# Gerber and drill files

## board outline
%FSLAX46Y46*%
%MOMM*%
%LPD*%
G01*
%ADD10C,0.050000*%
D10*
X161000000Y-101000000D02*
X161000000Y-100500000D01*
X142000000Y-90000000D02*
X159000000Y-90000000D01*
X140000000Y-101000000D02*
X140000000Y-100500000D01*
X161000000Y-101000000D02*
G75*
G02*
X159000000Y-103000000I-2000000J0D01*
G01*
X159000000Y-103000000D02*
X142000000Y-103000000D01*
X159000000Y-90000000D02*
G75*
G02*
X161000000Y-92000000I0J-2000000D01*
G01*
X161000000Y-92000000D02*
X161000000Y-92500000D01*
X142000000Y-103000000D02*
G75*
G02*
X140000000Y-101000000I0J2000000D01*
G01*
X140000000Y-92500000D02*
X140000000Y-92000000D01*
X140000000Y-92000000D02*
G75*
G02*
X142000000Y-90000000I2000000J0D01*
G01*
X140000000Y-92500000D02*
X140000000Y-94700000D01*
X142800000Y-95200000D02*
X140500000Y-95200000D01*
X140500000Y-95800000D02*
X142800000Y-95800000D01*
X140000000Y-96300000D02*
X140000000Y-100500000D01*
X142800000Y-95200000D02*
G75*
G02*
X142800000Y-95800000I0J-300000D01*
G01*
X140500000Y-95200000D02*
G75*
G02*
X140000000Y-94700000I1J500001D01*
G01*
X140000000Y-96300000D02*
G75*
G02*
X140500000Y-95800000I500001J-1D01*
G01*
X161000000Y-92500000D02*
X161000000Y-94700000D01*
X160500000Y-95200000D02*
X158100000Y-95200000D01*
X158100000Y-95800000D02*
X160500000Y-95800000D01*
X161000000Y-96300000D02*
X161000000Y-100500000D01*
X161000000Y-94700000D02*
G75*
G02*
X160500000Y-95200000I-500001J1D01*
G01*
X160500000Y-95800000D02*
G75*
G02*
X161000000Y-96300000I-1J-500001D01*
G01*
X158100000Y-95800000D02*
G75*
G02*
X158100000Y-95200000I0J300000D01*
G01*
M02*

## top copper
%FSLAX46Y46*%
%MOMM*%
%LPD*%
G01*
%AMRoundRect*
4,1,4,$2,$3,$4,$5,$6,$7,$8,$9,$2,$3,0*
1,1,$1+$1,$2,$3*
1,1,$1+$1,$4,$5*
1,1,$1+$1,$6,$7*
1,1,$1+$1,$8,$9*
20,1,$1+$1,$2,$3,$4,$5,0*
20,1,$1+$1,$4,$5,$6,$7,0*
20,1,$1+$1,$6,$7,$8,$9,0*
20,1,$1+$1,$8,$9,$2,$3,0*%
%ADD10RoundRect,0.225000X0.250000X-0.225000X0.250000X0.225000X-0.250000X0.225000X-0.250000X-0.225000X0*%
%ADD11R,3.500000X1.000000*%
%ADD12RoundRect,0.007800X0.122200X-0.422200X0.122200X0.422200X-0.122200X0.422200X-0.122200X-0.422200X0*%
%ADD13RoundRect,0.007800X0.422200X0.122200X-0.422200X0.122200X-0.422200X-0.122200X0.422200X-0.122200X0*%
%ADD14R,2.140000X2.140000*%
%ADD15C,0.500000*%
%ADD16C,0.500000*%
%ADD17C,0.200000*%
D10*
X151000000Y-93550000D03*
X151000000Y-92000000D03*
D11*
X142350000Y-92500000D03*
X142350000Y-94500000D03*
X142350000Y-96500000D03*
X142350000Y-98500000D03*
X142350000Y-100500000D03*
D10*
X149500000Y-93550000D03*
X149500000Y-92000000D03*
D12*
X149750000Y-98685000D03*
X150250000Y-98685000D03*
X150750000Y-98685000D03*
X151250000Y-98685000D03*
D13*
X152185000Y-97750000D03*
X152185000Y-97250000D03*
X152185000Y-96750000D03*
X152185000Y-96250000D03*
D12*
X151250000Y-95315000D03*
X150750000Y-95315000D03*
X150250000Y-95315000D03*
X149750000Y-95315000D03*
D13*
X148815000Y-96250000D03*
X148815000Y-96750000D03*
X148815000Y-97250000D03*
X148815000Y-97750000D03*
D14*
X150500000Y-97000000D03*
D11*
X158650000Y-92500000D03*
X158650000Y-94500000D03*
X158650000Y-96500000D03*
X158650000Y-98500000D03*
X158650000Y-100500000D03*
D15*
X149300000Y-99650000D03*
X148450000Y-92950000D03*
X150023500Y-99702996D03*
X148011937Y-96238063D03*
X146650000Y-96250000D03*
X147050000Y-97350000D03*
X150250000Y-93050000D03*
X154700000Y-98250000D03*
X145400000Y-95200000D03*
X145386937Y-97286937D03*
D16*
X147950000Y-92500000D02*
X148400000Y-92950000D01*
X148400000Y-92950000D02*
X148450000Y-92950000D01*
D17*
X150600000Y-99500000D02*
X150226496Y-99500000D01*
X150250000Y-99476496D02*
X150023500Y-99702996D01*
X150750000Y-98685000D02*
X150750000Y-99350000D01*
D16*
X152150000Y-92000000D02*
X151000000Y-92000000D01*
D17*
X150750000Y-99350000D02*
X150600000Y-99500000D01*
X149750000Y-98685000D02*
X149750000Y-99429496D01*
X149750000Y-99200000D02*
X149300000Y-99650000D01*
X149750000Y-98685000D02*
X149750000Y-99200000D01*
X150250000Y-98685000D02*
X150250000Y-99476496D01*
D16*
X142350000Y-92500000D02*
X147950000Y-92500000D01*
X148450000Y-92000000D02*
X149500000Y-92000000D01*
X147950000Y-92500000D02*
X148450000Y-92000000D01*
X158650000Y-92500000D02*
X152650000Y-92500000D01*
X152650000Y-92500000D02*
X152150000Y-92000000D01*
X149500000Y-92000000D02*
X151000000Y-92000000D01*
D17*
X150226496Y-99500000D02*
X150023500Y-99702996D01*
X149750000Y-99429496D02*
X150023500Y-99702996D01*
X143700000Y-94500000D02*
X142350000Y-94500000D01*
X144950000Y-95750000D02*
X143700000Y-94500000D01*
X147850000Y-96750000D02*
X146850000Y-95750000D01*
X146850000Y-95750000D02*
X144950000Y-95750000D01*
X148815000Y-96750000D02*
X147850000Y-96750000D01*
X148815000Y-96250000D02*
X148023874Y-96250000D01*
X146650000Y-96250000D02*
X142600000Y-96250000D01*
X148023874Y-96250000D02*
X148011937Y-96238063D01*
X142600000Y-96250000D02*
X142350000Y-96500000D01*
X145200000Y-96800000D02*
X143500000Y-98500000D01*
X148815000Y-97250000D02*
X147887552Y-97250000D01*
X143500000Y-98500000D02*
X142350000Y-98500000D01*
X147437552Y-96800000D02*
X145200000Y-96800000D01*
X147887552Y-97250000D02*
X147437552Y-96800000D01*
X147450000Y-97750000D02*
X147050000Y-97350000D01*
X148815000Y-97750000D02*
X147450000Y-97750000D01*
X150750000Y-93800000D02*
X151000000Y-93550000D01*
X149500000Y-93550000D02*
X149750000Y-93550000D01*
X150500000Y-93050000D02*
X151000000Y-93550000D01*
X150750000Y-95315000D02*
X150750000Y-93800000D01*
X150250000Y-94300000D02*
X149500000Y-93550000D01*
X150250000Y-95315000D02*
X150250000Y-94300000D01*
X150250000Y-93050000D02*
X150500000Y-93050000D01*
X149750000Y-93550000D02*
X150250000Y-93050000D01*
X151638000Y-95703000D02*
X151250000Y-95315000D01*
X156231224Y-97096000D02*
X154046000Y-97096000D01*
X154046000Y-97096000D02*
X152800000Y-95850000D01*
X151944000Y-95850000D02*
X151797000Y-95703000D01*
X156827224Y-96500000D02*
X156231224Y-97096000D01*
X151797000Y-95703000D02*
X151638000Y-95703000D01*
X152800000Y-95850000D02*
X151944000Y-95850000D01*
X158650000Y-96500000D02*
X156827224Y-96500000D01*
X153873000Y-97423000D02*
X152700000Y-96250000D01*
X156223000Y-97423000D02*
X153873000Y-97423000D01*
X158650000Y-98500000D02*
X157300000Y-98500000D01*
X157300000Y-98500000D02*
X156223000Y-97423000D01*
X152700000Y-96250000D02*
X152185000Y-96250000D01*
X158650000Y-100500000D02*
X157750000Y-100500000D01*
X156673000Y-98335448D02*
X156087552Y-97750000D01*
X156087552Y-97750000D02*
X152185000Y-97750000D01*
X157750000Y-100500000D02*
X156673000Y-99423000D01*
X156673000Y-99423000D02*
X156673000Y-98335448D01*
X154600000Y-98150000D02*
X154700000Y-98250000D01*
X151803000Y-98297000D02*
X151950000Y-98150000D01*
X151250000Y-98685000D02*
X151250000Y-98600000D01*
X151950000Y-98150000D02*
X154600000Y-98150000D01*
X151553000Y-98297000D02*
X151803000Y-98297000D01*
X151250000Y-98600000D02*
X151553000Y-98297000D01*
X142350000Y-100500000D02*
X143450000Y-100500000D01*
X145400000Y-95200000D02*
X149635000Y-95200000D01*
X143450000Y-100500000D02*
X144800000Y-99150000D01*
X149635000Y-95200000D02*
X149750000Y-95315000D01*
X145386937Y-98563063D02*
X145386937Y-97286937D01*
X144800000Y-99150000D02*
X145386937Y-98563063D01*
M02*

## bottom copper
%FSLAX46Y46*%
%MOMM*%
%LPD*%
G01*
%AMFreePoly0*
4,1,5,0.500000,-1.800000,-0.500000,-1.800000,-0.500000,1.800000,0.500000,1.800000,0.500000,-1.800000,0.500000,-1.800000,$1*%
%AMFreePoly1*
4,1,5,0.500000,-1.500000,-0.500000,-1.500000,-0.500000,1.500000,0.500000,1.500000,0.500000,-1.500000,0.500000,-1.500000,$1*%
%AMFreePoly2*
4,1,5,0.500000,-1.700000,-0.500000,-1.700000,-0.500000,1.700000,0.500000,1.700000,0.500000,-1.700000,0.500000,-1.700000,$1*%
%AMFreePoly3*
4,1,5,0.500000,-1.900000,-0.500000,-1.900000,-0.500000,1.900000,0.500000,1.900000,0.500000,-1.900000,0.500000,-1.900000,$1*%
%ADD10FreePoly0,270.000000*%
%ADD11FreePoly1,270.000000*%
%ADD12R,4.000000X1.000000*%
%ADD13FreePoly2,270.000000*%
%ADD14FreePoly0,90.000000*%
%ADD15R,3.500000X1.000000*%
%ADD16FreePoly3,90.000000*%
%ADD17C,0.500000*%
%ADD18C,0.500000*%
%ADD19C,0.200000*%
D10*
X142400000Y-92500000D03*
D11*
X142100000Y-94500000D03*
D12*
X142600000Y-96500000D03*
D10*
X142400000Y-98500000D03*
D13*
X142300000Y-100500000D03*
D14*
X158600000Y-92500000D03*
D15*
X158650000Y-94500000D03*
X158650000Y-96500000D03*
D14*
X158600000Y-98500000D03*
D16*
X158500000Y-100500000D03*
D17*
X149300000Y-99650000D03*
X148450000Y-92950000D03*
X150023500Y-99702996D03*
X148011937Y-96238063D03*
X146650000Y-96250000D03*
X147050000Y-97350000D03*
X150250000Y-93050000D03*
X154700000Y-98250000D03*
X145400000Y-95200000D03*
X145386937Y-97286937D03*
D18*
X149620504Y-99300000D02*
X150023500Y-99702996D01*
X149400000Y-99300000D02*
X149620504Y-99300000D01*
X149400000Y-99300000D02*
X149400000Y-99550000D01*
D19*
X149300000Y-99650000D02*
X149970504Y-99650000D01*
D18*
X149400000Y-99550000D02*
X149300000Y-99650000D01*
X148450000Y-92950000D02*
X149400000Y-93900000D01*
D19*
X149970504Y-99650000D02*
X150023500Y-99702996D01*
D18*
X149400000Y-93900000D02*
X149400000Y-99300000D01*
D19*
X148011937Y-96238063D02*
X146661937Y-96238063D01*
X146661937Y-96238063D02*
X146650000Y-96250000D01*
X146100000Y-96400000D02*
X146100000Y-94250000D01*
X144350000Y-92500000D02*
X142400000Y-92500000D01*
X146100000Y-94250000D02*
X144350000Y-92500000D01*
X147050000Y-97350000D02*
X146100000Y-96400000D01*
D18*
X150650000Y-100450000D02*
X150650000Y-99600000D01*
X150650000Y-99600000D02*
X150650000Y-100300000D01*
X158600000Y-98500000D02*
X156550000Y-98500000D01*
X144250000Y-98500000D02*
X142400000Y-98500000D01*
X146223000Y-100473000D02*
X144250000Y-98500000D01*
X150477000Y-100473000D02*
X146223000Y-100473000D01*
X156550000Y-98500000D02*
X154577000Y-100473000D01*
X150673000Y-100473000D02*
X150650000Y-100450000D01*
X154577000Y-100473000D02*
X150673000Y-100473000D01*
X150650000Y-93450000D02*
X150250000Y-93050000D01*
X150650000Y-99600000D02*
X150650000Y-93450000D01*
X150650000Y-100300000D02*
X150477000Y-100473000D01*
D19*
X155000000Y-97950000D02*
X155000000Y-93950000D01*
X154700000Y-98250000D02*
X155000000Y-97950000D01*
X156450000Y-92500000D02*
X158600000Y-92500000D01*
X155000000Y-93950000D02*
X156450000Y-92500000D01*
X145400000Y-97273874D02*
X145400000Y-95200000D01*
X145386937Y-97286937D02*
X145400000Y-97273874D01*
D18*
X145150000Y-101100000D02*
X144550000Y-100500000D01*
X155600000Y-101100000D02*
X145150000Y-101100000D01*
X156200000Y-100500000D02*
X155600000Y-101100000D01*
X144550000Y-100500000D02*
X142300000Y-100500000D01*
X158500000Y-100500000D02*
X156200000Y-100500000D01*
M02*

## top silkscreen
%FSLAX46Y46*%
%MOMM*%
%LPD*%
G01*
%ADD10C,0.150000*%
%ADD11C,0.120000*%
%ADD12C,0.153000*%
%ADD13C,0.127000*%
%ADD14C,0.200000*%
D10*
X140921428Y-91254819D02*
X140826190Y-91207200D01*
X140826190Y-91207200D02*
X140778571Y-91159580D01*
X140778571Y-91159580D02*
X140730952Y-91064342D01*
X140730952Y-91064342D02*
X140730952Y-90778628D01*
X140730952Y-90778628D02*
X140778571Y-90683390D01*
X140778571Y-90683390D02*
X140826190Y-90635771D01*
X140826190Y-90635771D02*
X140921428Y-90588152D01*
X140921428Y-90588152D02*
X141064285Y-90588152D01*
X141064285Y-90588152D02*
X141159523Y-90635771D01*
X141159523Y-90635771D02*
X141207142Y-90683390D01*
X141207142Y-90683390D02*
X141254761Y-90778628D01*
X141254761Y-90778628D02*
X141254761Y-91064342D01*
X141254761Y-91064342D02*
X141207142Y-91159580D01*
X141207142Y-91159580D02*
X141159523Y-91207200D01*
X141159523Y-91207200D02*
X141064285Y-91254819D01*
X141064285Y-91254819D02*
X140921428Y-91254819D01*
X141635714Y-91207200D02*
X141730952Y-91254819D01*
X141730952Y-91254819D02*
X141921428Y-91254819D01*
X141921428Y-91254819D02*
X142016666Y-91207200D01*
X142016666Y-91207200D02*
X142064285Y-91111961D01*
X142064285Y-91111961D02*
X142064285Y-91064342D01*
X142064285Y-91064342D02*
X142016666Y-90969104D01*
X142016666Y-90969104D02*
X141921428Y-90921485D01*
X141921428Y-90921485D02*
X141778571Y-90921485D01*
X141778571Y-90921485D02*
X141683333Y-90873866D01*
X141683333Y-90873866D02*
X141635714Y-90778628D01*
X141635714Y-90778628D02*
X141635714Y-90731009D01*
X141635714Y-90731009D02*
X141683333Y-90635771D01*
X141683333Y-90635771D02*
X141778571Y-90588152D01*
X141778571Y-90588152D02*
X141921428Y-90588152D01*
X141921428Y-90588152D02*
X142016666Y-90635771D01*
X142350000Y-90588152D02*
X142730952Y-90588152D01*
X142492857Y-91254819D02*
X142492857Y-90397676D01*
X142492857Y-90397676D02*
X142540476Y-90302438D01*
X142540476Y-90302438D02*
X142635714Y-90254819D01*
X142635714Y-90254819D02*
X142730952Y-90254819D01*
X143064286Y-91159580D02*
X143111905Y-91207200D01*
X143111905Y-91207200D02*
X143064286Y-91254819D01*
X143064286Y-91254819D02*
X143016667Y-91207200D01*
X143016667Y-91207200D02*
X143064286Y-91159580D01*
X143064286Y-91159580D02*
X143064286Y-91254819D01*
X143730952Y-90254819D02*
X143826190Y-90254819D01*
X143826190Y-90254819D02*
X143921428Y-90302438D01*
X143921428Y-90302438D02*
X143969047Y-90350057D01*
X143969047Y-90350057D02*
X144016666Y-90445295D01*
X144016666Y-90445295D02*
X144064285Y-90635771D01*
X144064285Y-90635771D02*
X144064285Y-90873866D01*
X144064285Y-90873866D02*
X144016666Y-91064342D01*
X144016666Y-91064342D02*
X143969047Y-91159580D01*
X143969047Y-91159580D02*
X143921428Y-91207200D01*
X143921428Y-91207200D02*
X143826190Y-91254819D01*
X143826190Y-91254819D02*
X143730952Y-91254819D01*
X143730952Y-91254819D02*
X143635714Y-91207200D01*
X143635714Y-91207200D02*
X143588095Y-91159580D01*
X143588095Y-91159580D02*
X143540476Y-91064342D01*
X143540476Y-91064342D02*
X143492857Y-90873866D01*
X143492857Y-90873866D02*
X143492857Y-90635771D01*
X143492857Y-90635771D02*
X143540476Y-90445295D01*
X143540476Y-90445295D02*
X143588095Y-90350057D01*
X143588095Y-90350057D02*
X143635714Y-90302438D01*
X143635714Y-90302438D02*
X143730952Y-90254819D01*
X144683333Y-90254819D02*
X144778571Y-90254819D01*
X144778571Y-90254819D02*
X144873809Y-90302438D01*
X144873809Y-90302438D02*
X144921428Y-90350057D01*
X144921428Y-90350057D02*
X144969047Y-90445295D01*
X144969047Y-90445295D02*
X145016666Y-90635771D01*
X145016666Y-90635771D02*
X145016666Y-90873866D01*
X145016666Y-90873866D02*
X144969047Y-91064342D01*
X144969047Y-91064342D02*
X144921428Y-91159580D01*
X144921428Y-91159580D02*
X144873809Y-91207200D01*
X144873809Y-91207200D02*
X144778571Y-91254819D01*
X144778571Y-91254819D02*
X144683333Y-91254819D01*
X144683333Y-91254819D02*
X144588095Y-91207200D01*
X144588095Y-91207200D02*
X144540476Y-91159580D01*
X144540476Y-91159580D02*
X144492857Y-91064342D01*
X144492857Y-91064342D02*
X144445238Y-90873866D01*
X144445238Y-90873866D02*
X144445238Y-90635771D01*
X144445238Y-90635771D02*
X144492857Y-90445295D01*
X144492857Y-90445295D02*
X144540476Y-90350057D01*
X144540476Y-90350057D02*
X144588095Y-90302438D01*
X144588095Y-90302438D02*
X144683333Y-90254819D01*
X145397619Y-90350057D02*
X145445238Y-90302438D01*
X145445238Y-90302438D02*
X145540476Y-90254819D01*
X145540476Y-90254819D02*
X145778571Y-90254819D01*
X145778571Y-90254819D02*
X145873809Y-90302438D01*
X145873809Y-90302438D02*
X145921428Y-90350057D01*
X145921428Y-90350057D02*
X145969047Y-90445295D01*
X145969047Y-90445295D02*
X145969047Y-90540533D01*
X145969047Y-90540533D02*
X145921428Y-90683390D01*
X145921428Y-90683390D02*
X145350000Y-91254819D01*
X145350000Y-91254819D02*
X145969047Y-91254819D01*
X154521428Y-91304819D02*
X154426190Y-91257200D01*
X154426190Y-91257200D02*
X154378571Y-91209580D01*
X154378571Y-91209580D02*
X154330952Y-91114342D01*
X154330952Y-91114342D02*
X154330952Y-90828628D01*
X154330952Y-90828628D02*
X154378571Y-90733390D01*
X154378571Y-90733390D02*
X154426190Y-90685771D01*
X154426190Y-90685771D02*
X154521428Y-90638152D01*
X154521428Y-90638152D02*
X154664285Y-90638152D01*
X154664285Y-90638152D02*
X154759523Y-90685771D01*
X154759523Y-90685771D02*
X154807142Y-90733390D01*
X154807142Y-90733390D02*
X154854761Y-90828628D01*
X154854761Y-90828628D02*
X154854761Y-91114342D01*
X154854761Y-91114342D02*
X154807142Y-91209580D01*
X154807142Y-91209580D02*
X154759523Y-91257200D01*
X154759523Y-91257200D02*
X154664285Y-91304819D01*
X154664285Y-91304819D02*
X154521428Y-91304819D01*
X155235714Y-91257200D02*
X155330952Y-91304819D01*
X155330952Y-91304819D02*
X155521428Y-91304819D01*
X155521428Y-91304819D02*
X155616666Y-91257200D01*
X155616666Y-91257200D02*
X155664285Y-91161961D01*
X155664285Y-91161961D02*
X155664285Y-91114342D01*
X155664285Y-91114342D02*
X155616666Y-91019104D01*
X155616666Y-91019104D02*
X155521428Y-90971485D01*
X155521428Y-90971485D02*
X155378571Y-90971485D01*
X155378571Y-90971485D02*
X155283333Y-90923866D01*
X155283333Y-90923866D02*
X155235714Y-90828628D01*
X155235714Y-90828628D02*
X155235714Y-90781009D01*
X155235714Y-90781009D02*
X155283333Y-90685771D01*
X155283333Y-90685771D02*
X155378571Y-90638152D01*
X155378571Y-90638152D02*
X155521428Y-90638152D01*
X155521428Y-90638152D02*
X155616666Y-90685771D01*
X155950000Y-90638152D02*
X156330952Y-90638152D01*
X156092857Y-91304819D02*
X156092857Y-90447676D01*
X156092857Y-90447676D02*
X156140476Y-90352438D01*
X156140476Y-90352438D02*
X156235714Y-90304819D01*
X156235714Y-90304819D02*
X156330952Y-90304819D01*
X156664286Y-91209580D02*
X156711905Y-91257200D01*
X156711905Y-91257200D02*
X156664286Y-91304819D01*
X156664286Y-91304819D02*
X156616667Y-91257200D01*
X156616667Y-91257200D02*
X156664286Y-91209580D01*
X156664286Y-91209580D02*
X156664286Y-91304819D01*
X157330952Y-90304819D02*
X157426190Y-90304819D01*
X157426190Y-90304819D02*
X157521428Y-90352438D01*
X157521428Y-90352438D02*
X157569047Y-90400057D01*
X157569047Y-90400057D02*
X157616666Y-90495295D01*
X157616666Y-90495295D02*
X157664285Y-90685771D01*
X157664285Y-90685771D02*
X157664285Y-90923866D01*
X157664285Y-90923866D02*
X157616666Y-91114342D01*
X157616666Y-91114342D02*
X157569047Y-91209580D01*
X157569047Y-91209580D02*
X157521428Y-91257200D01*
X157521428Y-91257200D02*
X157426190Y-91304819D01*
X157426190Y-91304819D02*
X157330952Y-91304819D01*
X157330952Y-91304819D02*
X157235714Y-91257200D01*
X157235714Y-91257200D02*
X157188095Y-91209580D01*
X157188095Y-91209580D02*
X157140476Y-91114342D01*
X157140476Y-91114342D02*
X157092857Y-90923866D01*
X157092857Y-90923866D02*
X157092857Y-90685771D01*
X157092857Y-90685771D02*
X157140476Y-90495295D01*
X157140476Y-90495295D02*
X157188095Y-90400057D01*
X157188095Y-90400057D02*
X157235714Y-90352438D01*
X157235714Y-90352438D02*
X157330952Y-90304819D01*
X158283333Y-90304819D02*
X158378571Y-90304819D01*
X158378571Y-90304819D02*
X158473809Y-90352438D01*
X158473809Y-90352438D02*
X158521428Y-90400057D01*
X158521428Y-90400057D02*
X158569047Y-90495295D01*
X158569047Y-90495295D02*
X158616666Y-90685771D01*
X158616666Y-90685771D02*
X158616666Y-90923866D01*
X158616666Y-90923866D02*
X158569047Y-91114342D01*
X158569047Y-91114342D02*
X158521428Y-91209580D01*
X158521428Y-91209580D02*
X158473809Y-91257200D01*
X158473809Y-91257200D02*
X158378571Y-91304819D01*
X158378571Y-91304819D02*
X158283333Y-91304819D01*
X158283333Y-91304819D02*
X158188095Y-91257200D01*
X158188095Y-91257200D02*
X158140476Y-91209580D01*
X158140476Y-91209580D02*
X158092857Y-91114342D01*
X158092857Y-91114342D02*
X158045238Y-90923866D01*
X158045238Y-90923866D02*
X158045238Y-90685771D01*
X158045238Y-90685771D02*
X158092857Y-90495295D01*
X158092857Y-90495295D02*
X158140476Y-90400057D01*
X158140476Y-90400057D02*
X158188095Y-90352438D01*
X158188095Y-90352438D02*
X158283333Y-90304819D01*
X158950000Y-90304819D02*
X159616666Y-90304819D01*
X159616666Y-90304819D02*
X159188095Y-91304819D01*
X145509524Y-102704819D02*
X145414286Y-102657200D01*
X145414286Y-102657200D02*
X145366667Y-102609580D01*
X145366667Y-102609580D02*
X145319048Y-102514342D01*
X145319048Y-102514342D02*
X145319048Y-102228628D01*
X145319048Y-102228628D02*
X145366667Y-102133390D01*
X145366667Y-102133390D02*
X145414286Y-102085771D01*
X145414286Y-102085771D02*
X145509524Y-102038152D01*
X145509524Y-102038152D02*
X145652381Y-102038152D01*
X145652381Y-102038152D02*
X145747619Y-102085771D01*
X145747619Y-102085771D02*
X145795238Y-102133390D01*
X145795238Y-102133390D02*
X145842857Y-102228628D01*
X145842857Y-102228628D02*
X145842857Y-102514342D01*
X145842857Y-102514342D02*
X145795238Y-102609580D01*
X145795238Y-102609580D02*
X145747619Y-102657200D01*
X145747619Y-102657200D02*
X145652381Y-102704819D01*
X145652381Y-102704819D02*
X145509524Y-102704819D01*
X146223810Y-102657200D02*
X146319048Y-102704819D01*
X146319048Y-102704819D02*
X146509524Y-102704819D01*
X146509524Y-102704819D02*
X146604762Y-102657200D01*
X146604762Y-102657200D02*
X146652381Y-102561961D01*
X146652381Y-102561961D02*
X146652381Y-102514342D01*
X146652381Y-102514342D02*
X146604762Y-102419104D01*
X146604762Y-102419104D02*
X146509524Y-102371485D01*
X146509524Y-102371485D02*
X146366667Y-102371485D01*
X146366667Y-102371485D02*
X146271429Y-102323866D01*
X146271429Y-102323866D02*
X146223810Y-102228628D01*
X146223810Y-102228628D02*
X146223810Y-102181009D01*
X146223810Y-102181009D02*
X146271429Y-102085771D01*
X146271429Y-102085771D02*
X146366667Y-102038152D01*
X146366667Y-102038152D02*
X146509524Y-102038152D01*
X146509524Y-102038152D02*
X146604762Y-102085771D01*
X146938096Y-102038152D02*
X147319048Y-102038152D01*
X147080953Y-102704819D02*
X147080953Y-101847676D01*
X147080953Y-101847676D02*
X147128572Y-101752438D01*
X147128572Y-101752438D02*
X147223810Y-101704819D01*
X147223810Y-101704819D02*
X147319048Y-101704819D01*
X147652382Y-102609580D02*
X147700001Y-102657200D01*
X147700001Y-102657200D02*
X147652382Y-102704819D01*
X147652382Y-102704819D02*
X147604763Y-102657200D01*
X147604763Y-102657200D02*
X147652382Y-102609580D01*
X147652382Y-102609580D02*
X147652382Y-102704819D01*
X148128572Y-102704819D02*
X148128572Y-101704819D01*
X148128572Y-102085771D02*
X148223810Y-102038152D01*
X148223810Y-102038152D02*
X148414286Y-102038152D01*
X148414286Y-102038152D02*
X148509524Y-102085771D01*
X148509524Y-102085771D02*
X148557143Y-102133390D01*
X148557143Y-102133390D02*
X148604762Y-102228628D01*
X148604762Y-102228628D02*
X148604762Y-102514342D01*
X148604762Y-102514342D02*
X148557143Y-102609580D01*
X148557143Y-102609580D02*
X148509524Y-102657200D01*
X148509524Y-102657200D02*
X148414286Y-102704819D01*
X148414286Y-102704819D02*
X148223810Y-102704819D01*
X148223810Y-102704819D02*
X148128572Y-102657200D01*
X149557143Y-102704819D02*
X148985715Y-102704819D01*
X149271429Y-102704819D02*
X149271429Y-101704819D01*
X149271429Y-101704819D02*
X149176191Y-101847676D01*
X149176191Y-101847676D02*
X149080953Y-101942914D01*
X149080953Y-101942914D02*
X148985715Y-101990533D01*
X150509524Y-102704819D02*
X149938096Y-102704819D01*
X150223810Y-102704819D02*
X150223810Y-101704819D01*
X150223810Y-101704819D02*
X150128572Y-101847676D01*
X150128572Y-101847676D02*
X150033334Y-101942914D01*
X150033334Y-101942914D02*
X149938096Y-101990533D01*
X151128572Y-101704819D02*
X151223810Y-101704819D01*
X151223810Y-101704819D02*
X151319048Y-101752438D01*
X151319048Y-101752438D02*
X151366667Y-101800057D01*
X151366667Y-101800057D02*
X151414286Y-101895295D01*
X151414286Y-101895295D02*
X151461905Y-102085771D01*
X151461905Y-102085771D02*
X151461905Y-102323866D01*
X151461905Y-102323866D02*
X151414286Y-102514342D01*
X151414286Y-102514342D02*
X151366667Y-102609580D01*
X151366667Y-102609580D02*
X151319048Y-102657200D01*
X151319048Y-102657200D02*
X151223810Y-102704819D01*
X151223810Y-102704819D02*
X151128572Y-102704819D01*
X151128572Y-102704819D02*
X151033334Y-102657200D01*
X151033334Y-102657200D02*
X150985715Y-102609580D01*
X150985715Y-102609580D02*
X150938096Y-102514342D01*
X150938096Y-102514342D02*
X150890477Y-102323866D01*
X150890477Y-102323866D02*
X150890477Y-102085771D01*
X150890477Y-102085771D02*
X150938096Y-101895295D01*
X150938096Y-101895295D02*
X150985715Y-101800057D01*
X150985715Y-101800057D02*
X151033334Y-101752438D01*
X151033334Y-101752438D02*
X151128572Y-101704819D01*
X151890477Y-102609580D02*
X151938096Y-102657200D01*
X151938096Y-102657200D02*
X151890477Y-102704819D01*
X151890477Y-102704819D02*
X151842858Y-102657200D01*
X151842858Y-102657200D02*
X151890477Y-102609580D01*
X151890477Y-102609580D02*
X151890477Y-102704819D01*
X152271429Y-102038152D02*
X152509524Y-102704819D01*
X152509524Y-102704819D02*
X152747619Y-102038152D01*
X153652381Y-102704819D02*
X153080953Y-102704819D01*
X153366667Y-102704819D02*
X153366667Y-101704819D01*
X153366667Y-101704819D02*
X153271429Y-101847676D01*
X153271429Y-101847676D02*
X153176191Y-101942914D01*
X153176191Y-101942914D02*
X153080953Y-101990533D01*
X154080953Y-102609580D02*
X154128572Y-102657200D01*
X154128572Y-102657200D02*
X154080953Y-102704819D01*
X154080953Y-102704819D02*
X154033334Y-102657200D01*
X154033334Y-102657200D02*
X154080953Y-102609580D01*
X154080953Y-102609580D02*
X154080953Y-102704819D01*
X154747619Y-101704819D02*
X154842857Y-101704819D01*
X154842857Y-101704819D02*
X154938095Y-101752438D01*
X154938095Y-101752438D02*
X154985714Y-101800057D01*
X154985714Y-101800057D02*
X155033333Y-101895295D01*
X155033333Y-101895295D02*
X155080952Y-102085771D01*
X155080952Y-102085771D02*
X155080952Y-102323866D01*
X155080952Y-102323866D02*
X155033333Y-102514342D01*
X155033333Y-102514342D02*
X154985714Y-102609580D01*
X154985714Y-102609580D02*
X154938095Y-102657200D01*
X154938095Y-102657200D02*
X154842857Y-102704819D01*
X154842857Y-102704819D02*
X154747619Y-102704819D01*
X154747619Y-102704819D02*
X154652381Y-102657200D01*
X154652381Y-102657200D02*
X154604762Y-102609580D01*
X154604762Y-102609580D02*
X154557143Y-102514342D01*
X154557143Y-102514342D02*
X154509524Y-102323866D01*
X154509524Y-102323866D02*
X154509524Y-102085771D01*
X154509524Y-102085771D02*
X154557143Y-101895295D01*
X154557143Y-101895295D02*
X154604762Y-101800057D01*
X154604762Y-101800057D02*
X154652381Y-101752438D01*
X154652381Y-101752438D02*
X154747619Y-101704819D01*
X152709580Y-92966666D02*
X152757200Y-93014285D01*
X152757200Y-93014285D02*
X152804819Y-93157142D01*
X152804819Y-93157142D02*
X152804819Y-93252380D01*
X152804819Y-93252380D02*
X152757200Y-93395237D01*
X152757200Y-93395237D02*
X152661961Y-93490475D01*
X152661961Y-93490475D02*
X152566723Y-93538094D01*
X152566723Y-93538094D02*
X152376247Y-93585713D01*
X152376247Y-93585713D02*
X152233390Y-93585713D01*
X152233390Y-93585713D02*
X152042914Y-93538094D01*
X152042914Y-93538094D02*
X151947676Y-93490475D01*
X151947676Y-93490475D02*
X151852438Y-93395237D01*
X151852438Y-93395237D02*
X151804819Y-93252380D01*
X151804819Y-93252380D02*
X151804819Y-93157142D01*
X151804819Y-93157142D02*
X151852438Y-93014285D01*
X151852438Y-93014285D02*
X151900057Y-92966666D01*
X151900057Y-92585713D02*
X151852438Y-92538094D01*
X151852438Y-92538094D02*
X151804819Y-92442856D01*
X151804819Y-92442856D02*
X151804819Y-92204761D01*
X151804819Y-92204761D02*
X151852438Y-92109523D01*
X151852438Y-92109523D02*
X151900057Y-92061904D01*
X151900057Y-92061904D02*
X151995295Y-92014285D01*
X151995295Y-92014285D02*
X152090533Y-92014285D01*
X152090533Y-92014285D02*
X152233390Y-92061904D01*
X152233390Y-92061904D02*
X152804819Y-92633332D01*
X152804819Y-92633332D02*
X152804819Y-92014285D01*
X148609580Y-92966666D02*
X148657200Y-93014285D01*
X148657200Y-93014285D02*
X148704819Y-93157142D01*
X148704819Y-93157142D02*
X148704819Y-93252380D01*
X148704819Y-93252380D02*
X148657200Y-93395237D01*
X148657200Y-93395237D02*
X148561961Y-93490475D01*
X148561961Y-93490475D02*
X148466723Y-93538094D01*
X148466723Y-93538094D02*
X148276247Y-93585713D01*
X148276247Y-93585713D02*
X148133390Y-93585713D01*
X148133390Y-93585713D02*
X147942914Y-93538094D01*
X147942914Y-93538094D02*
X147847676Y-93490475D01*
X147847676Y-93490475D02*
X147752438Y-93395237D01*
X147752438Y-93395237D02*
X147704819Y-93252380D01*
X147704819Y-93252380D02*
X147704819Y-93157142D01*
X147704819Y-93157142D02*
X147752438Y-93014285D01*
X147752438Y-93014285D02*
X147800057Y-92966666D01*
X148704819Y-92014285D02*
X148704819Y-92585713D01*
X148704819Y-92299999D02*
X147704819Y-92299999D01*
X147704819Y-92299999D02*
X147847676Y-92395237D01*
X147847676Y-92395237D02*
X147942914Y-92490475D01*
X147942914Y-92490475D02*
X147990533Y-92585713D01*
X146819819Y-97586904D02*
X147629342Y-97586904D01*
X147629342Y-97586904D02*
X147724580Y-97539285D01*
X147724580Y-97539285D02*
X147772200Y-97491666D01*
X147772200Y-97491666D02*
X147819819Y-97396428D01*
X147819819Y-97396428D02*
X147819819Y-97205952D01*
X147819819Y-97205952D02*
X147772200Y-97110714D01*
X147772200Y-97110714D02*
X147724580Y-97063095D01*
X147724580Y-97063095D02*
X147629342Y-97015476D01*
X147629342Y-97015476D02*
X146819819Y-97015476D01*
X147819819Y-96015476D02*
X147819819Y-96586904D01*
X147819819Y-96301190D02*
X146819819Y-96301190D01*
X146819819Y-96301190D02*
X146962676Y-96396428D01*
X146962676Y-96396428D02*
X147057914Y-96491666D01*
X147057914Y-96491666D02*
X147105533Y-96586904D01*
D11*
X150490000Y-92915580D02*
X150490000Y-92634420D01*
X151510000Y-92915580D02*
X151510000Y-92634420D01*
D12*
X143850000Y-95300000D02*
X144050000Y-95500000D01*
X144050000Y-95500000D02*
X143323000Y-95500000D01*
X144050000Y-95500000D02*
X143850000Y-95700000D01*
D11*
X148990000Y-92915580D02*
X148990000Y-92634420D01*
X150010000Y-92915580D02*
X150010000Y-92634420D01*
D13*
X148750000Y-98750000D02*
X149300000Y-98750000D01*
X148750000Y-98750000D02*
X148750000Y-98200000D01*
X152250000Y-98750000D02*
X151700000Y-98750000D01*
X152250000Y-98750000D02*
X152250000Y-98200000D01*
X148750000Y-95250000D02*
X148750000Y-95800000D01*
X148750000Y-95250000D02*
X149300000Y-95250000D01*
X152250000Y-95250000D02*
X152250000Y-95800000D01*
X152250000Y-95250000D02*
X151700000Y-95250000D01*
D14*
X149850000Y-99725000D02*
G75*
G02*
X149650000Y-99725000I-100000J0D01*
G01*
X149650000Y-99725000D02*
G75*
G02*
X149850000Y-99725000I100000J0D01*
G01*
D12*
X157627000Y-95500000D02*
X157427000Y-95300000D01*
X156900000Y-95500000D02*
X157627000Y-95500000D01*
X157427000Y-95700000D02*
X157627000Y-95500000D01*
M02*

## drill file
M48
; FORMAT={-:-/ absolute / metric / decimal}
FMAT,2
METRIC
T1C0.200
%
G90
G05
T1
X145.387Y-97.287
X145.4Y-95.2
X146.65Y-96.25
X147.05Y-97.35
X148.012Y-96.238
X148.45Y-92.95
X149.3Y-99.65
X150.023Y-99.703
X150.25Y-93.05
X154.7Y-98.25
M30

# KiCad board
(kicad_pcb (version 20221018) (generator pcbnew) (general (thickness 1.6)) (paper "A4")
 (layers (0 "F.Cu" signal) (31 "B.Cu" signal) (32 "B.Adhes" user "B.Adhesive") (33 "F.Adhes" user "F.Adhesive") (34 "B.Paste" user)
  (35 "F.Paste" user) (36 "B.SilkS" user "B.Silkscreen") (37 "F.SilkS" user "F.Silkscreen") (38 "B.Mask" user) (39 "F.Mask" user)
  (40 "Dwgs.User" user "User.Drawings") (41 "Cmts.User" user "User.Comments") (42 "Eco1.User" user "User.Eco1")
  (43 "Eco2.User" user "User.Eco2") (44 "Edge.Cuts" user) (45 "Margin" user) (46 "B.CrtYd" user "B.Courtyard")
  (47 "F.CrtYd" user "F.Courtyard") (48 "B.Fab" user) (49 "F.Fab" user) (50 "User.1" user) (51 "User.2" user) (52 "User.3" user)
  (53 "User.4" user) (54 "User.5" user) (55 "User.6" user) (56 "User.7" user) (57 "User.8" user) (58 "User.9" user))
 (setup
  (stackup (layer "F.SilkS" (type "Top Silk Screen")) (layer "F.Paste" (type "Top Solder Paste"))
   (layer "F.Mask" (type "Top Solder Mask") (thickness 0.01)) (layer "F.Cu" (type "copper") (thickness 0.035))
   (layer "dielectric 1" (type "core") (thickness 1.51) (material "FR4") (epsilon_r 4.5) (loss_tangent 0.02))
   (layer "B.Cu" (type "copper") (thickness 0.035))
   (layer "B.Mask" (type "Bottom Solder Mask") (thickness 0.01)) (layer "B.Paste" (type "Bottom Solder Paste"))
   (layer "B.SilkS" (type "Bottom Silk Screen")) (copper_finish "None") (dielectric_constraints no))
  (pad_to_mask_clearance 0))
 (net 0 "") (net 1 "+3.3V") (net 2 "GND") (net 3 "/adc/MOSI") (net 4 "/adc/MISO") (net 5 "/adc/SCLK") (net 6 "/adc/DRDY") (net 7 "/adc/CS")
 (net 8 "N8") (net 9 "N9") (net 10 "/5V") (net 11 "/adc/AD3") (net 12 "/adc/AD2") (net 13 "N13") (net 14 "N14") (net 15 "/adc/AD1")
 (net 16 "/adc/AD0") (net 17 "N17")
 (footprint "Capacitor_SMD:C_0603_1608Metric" (layer "F.Cu") (at 151 92.775 90)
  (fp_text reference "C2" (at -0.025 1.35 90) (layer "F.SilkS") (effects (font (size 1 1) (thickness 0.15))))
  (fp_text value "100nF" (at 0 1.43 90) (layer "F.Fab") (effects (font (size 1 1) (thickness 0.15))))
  (fp_line (start -0.14058 -0.51) (end 0.14058 -0.51) (stroke (width 0.12) (type solid)) (layer "F.SilkS"))
  (fp_line (start -0.14058 0.51) (end 0.14058 0.51) (stroke (width 0.12) (type solid)) (layer "F.SilkS"))
  (pad "1" smd roundrect (at -0.775 0 90) (size 0.9 0.95) (layers "F.Cu" "F.Paste" "F.Mask") (roundrect_rratio 0.25) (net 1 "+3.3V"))
  (pad "2" smd roundrect (at 0.775 0 90) (size 0.9 0.95) (layers "F.Cu" "F.Paste" "F.Mask") (roundrect_rratio 0.25) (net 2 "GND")))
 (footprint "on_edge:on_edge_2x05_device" (layer "F.Cu") (at 140 96.5 -90)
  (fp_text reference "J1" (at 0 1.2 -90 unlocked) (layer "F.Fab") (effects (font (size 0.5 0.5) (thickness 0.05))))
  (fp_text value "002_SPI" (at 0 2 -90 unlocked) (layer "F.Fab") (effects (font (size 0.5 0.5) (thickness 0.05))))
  (fp_line (start -1.2 -3.85) (end -1 -4.05) (stroke (width 0.153) (type solid)) (layer "F.SilkS"))
  (fp_line (start -1 -4.05) (end -1 -3.323) (stroke (width 0.153) (type solid)) (layer "F.SilkS"))
  (fp_line (start -1 -4.05) (end -0.8 -3.85) (stroke (width 0.153) (type solid)) (layer "F.SilkS"))
  (fp_line (start -4 0) (end -1.8 0) (stroke (width 0.05) (type solid)) (layer "Edge.Cuts"))
  (fp_line (start -1.3 -2.8) (end -1.3 -0.5) (stroke (width 0.05) (type solid)) (layer "Edge.Cuts"))
  (fp_line (start -0.7 -0.5) (end -0.7 -2.8) (stroke (width 0.05) (type solid)) (layer "Edge.Cuts"))
  (fp_line (start -0.2 0) (end 4 0) (stroke (width 0.05) (type solid)) (layer "Edge.Cuts"))
  (fp_arc (start -1.3 -2.8) (mid -1 -3.1) (end -0.7 -2.8) (stroke (width 0.05) (type solid)) (layer "Edge.Cuts"))
  (fp_arc (start -1.3 -0.5) (mid -1.446447 -0.146447) (end -1.8 0) (stroke (width 0.05) (type solid)) (layer "Edge.Cuts"))
  (fp_arc (start -0.2 0) (mid -0.553553 -0.146447) (end -0.7 -0.5) (stroke (width 0.05) (type solid)) (layer "Edge.Cuts"))
  (pad "1" smd rect (at -4 -2.35 90) (size 1 3.5) (layers "F.Cu" "F.Mask") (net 2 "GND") (zone_connect 0))
  (pad "2" smd rect (at -2 -2.35 270) (size 1 3.5) (layers "F.Cu" "F.Mask") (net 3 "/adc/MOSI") (zone_connect 0))
  (pad "3" smd rect (at 0 -2.35 270) (size 1 3.5) (layers "F.Cu" "F.Mask") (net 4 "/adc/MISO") (zone_connect 0))
  (pad "4" smd rect (at 2 -2.35 90) (size 1 3.5) (layers "F.Cu" "F.Mask") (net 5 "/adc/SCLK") (zone_connect 0))
  (pad "5" smd rect (at 4 -2.35 90) (size 1 3.5) (layers "F.Cu" "F.Mask") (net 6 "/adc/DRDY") (zone_connect 0))
  (pad "6" smd custom (at -4 -2.4 270) (size 1 3.6) (layers "B.Cu" "B.Mask") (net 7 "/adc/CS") (zone_connect 0)
   (options (clearance outline) (anchor rect)) (primitives))
  (pad "7" smd custom (at -2 -2.1 270) (size 1 3) (layers "B.Cu" "B.Mask") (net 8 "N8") (zone_connect 0)
   (options (clearance outline) (anchor rect)) (primitives))
  (pad "8" smd rect (at 0 -2.6 270) (size 1 4) (layers "B.Cu" "B.Mask") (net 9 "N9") (zone_connect 0))
  (pad "9" smd custom (at 2 -2.4 270) (size 1 3.6) (layers "B.Cu" "B.Mask") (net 1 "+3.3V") (zone_connect 0)
   (options (clearance outline) (anchor rect)) (primitives))
  (pad "10" smd custom (at 4 -2.3 270) (size 1 3.4) (layers "B.Cu" "B.Mask") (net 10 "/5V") (zone_connect 0)
   (options (clearance outline) (anchor rect)) (primitives))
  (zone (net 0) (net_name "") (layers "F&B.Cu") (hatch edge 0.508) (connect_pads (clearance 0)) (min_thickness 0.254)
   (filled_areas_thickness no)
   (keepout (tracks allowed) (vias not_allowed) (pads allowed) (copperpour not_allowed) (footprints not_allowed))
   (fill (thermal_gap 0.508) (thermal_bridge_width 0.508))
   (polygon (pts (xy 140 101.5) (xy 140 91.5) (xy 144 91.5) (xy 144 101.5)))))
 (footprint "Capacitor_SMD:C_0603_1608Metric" (layer "F.Cu") (at 149.5 92.775 90)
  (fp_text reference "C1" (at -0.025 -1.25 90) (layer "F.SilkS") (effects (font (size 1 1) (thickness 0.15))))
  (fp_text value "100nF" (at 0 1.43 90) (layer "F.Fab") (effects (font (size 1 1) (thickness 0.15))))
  (fp_line (start -0.14058 -0.51) (end 0.14058 -0.51) (stroke (width 0.12) (type solid)) (layer "F.SilkS"))
  (fp_line (start -0.14058 0.51) (end 0.14058 0.51) (stroke (width 0.12) (type solid)) (layer "F.SilkS"))
  (pad "1" smd roundrect (at -0.775 0 90) (size 0.9 0.95) (layers "F.Cu" "F.Paste" "F.Mask") (roundrect_rratio 0.25) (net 1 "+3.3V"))
  (pad "2" smd roundrect (at 0.775 0 90) (size 0.9 0.95) (layers "F.Cu" "F.Paste" "F.Mask") (roundrect_rratio 0.25) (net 2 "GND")))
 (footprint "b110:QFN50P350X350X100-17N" (layer "F.Cu") (at 150.5 97 90)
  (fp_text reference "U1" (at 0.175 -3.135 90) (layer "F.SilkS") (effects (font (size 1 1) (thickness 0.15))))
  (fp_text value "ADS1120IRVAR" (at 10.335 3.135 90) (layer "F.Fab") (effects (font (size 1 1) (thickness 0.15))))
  (fp_line (start -1.75 -1.75) (end -1.75 -1.2) (stroke (width 0.127) (type solid)) (layer "F.SilkS"))
  (fp_line (start -1.75 -1.75) (end -1.2 -1.75) (stroke (width 0.127) (type solid)) (layer "F.SilkS"))
  (fp_line (start -1.75 1.75) (end -1.75 1.2) (stroke (width 0.127) (type solid)) (layer "F.SilkS"))
  (fp_line (start -1.75 1.75) (end -1.2 1.75) (stroke (width 0.127) (type solid)) (layer "F.SilkS"))
  (fp_line (start 1.75 -1.75) (end 1.2 -1.75) (stroke (width 0.127) (type solid)) (layer "F.SilkS"))
  (fp_line (start 1.75 -1.75) (end 1.75 -1.2) (stroke (width 0.127) (type solid)) (layer "F.SilkS"))
  (fp_line (start 1.75 1.75) (end 1.2 1.75) (stroke (width 0.127) (type solid)) (layer "F.SilkS"))
  (fp_line (start 1.75 1.75) (end 1.75 1.2) (stroke (width 0.127) (type solid)) (layer "F.SilkS"))
  (fp_circle (center -2.725 -0.75) (end -2.625 -0.75) (stroke (width 0.2) (type solid)) (fill none) (layer "F.SilkS"))
  (pad "1" smd roundrect (at -1.685 -0.75 90) (size 0.86 0.26) (layers "F.Cu" "F.Paste" "F.Mask") (roundrect_rratio 0.03) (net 2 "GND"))
  (pad "2" smd roundrect (at -1.685 -0.25 90) (size 0.86 0.26) (layers "F.Cu" "F.Paste" "F.Mask") (roundrect_rratio 0.03) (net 2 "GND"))
  (pad "3" smd roundrect (at -1.685 0.25 90) (size 0.86 0.26) (layers "F.Cu" "F.Paste" "F.Mask") (roundrect_rratio 0.03) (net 2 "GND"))
  (pad "4" smd roundrect (at -1.685 0.75 90) (size 0.86 0.26) (layers "F.Cu" "F.Paste" "F.Mask") (roundrect_rratio 0.03) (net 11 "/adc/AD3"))
  (pad "5" smd roundrect (at -0.75 1.685 180) (size 0.86 0.26) (layers "F.Cu" "F.Paste" "F.Mask") (roundrect_rratio 0.03)
   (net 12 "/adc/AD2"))
  (pad "6" smd roundrect (at -0.25 1.685 180) (size 0.86 0.26) (layers "F.Cu" "F.Paste" "F.Mask") (roundrect_rratio 0.03) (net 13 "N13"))
  (pad "7" smd roundrect (at 0.25 1.685 180) (size 0.86 0.26) (layers "F.Cu" "F.Paste" "F.Mask") (roundrect_rratio 0.03) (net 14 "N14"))
  (pad "8" smd roundrect (at 0.75 1.685 180) (size 0.86 0.26) (layers "F.Cu" "F.Paste" "F.Mask") (roundrect_rratio 0.03) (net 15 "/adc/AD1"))
  (pad "9" smd roundrect (at 1.685 0.75 90) (size 0.86 0.26) (layers "F.Cu" "F.Paste" "F.Mask") (roundrect_rratio 0.03) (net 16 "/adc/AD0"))
  (pad "10" smd roundrect (at 1.685 0.25 90) (size 0.86 0.26) (layers "F.Cu" "F.Paste" "F.Mask") (roundrect_rratio 0.03) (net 1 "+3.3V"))
  (pad "11" smd roundrect (at 1.685 -0.25 90) (size 0.86 0.26) (layers "F.Cu" "F.Paste" "F.Mask") (roundrect_rratio 0.03) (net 1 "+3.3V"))
  (pad "12" smd roundrect (at 1.685 -0.75 90) (size 0.86 0.26) (layers "F.Cu" "F.Paste" "F.Mask") (roundrect_rratio 0.03)
   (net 6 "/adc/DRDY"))
  (pad "13" smd roundrect (at 0.75 -1.685 180) (size 0.86 0.26) (layers "F.Cu" "F.Paste" "F.Mask") (roundrect_rratio 0.03)
   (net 4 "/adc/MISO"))
  (pad "14" smd roundrect (at 0.25 -1.685 180) (size 0.86 0.26) (layers "F.Cu" "F.Paste" "F.Mask") (roundrect_rratio 0.03)
   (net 3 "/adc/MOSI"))
  (pad "15" smd roundrect (at -0.25 -1.685 180) (size 0.86 0.26) (layers "F.Cu" "F.Paste" "F.Mask") (roundrect_rratio 0.03)
   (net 5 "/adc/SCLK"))
  (pad "16" smd roundrect (at -0.75 -1.685 180) (size 0.86 0.26) (layers "F.Cu" "F.Paste" "F.Mask") (roundrect_rratio 0.03)
   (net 7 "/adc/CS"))
  (pad "17" smd rect (at 0 0 90) (size 2.14 2.14) (layers "F.Cu" "F.Mask")))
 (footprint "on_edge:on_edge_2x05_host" (layer "F.Cu") (at 161 96.5 -90)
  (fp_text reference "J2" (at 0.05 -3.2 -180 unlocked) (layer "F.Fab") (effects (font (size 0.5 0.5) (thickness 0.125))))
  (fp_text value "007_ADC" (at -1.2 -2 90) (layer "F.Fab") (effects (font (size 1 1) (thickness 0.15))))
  (fp_line (start -1 3.373) (end -1.2 3.573) (stroke (width 0.153) (type solid)) (layer "F.SilkS"))
  (fp_line (start -1 4.1) (end -1 3.373) (stroke (width 0.153) (type solid)) (layer "F.SilkS"))
  (fp_line (start -0.8 3.573) (end -1 3.373) (stroke (width 0.153) (type solid)) (layer "F.SilkS"))
  (fp_line (start -4 0) (end -1.8 0) (stroke (width 0.05) (type solid)) (layer "Edge.Cuts"))
  (fp_line (start -1.3 0.5) (end -1.3 2.9) (stroke (width 0.05) (type solid)) (layer "Edge.Cuts"))
  (fp_line (start -0.7 2.9) (end -0.7 0.5) (stroke (width 0.05) (type solid)) (layer "Edge.Cuts"))
  (fp_line (start -0.2 0) (end 4 0) (stroke (width 0.05) (type solid)) (layer "Edge.Cuts"))
  (fp_arc (start -1.8 0) (mid -1.446447 0.146447) (end -1.3 0.5) (stroke (width 0.05) (type solid)) (layer "Edge.Cuts"))
  (fp_arc (start -0.7 0.5) (mid -0.553553 0.146447) (end -0.2 0) (stroke (width 0.05) (type solid)) (layer "Edge.Cuts"))
  (fp_arc (start -0.7 2.9) (mid -1 3.2) (end -1.3 2.9) (stroke (width 0.05) (type solid)) (layer "Edge.Cuts"))
  (pad "1" smd rect (at -4 2.35 270) (size 1 3.5) (layers "F.Cu" "F.Mask") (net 2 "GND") (zone_connect 0))
  (pad "2" smd rect (at -2 2.35 270) (size 1 3.5) (layers "F.Cu" "F.Mask") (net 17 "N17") (zone_connect 0))
  (pad "3" smd rect (at 0 2.35 270) (size 1 3.5) (layers "F.Cu" "F.Mask") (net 16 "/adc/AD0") (zone_connect 0))
  (pad "4" smd rect (at 2 2.35 270) (size 1 3.5) (layers "F.Cu" "F.Mask") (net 15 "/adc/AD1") (zone_connect 0))
  (pad "5" smd rect (at 4 2.35 270) (size 1 3.5) (layers "F.Cu" "F.Mask") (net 12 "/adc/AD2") (zone_connect 0))
  (pad "6" smd custom (at -4 2.4 90) (size 1 3.6) (layers "B.Cu" "B.Mask") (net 11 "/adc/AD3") (zone_connect 0)
   (options (clearance outline) (anchor rect)) (primitives))
  (pad "7" smd rect (at -2 2.35 90) (size 1 3.5) (layers "B.Cu" "B.Mask") (zone_connect 0))
  (pad "8" smd rect (at 0 2.35 90) (size 1 3.5) (layers "B.Cu" "B.Mask") (zone_connect 0))
  (pad "9" smd custom (at 2 2.4 90) (size 1 3.6) (layers "B.Cu" "B.Mask") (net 1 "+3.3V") (zone_connect 0)
   (options (clearance outline) (anchor rect)) (primitives))
  (pad "10" smd custom (at 4 2.5 90) (size 1 3.8) (layers "B.Cu" "B.Mask") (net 10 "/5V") (zone_connect 0)
   (options (clearance outline) (anchor rect)) (primitives))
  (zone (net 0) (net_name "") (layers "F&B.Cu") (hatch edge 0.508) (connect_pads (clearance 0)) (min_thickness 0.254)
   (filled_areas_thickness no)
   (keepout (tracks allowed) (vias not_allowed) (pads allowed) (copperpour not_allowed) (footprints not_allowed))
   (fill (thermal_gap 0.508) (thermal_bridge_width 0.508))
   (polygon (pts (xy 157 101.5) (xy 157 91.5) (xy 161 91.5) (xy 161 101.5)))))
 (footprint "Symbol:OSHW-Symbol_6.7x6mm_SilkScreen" (layer "B.Cu") (at 150.6 98.4 180)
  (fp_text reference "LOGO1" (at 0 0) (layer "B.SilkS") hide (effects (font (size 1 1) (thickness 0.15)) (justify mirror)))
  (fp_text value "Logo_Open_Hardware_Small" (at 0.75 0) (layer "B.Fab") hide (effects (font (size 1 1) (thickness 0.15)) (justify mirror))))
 (gr_line (start 161 101) (end 161 100.5) (stroke (width 0.05) (type solid)) (layer "Edge.Cuts"))
 (gr_line (start 142 90) (end 159 90) (stroke (width 0.05) (type solid)) (layer "Edge.Cuts"))
 (gr_line (start 140 101) (end 140 100.5) (stroke (width 0.05) (type solid)) (layer "Edge.Cuts"))
 (gr_arc (start 161 101) (mid 160.414214 102.414214) (end 159 103) (stroke (width 0.05) (type solid)) (layer "Edge.Cuts"))
 (gr_line (start 159 103) (end 142 103) (stroke (width 0.05) (type solid)) (layer "Edge.Cuts"))
 (gr_arc (start 159 90) (mid 160.414214 90.585786) (end 161 92) (stroke (width 0.05) (type solid)) (layer "Edge.Cuts"))
 (gr_line (start 161 92) (end 161 92.5) (stroke (width 0.05) (type solid)) (layer "Edge.Cuts"))
 (gr_arc (start 142 103) (mid 140.585786 102.414214) (end 140 101) (stroke (width 0.05) (type solid)) (layer "Edge.Cuts"))
 (gr_line (start 140 92.5) (end 140 92) (stroke (width 0.05) (type solid)) (layer "Edge.Cuts"))
 (gr_arc (start 140 92) (mid 140.585786 90.585786) (end 142 90) (stroke (width 0.05) (type solid)) (layer "Edge.Cuts"))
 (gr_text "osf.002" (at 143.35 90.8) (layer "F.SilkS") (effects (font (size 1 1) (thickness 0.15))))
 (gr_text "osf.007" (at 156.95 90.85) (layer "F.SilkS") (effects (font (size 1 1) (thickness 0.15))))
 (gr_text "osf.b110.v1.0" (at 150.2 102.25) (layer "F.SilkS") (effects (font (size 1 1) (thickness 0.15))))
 (segment (start 147.95 92.5) (end 148.4 92.95) (width 0.5) (layer "F.Cu") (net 2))
 (segment (start 148.4 92.95) (end 148.45 92.95) (width 0.5) (layer "F.Cu") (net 2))
 (segment (start 150.6 99.5) (end 150.226496 99.5) (width 0.2) (layer "F.Cu") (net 2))
 (segment (start 150.25 99.476496) (end 150.0235 99.702996) (width 0.2) (layer "F.Cu") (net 2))
 (segment (start 150.75 98.685) (end 150.75 99.35) (width 0.2) (layer "F.Cu") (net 2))
 (segment (start 152.15 92) (end 151 92) (width 0.5) (layer "F.Cu") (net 2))
 (segment (start 150.75 99.35) (end 150.6 99.5) (width 0.2) (layer "F.Cu") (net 2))
 (segment (start 149.75 98.685) (end 149.75 99.429496) (width 0.2) (layer "F.Cu") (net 2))
 (segment (start 149.75 99.2) (end 149.3 99.65) (width 0.2) (layer "F.Cu") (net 2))
 (segment (start 149.75 98.685) (end 149.75 99.2) (width 0.2) (layer "F.Cu") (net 2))
 (segment (start 150.25 98.685) (end 150.25 99.476496) (width 0.2) (layer "F.Cu") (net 2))
 (segment (start 142.35 92.5) (end 147.95 92.5) (width 0.5) (layer "F.Cu") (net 2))
 (segment (start 148.45 92) (end 149.5 92) (width 0.5) (layer "F.Cu") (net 2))
 (segment (start 147.95 92.5) (end 148.45 92) (width 0.5) (layer "F.Cu") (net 2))
 (segment (start 158.65 92.5) (end 152.65 92.5) (width 0.5) (layer "F.Cu") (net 2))
 (segment (start 152.65 92.5) (end 152.15 92) (width 0.5) (layer "F.Cu") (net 2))
 (segment (start 149.5 92) (end 151 92) (width 0.5) (layer "F.Cu") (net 2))
 (segment (start 150.226496 99.5) (end 150.0235 99.702996) (width 0.2) (layer "F.Cu") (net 2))
 (segment (start 149.75 99.429496) (end 150.0235 99.702996) (width 0.2) (layer "F.Cu") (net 2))
 (via (at 149.3 99.65) (size 0.5) (drill 0.2) (layers "F.Cu" "B.Cu") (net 2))
 (via (at 148.45 92.95) (size 0.5) (drill 0.2) (layers "F.Cu" "B.Cu") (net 2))
 (via (at 150.0235 99.702996) (size 0.5) (drill 0.2) (layers "F.Cu" "B.Cu") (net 2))
 (segment (start 149.620504 99.3) (end 150.0235 99.702996) (width 0.5) (layer "B.Cu") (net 2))
 (segment (start 149.4 99.3) (end 149.620504 99.3) (width 0.5) (layer "B.Cu") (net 2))
 (segment (start 149.4 99.3) (end 149.4 99.55) (width 0.5) (layer "B.Cu") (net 2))
 (segment (start 149.3 99.65) (end 149.970504 99.65) (width 0.2) (layer "B.Cu") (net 2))
 (segment (start 149.4 99.55) (end 149.3 99.65) (width 0.5) (layer "B.Cu") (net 2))
 (segment (start 148.45 92.95) (end 149.4 93.9) (width 0.5) (layer "B.Cu") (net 2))
 (segment (start 149.970504 99.65) (end 150.0235 99.702996) (width 0.2) (layer "B.Cu") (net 2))
 (segment (start 149.4 93.9) (end 149.4 99.3) (width 0.5) (layer "B.Cu") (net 2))
 (segment (start 143.7 94.5) (end 142.35 94.5) (width 0.2) (layer "F.Cu") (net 3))
 (segment (start 144.95 95.75) (end 143.7 94.5) (width 0.2) (layer "F.Cu") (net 3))
 (segment (start 147.85 96.75) (end 146.85 95.75) (width 0.2) (layer "F.Cu") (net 3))
 (segment (start 146.85 95.75) (end 144.95 95.75) (width 0.2) (layer "F.Cu") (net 3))
 (segment (start 148.815 96.75) (end 147.85 96.75) (width 0.2) (layer "F.Cu") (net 3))
 (segment (start 148.815 96.25) (end 148.023874 96.25) (width 0.2) (layer "F.Cu") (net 4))
 (segment (start 146.65 96.25) (end 142.6 96.25) (width 0.2) (layer "F.Cu") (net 4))
 (segment (start 148.023874 96.25) (end 148.011937 96.238063) (width 0.2) (layer "F.Cu") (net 4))
 (segment (start 142.6 96.25) (end 142.35 96.5) (width 0.2) (layer "F.Cu") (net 4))
 (via (at 148.011937 96.238063) (size 0.5) (drill 0.2) (layers "F.Cu" "B.Cu") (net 4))
 (via (at 146.65 96.25) (size 0.5) (drill 0.2) (layers "F.Cu" "B.Cu") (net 4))
 (segment (start 148.011937 96.238063) (end 146.661937 96.238063) (width 0.2) (layer "B.Cu") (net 4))
 (segment (start 146.661937 96.238063) (end 146.65 96.25) (width 0.2) (layer "B.Cu") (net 4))
 (segment (start 145.2 96.8) (end 143.5 98.5) (width 0.2) (layer "F.Cu") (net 5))
 (segment (start 148.815 97.25) (end 147.887552 97.25) (width 0.2) (layer "F.Cu") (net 5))
 (segment (start 143.5 98.5) (end 142.35 98.5) (width 0.2) (layer "F.Cu") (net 5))
 (segment (start 147.437552 96.8) (end 145.2 96.8) (width 0.2) (layer "F.Cu") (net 5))
 (segment (start 147.887552 97.25) (end 147.437552 96.8) (width 0.2) (layer "F.Cu") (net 5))
 (segment (start 147.45 97.75) (end 147.05 97.35) (width 0.2) (layer "F.Cu") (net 7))
 (segment (start 148.815 97.75) (end 147.45 97.75) (width 0.2) (layer "F.Cu") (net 7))
 (via (at 147.05 97.35) (size 0.5) (drill 0.2) (layers "F.Cu" "B.Cu") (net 7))
 (segment (start 146.1 96.4) (end 146.1 94.25) (width 0.2) (layer "B.Cu") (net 7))
 (segment (start 144.35 92.5) (end 142.4 92.5) (width 0.2) (layer "B.Cu") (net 7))
 (segment (start 146.1 94.25) (end 144.35 92.5) (width 0.2) (layer "B.Cu") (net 7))
 (segment (start 147.05 97.35) (end 146.1 96.4) (width 0.2) (layer "B.Cu") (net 7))
 (segment (start 150.75 93.8) (end 151 93.55) (width 0.2) (layer "F.Cu") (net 1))
 (segment (start 149.5 93.55) (end 149.75 93.55) (width 0.2) (layer "F.Cu") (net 1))
 (segment (start 150.5 93.05) (end 151 93.55) (width 0.2) (layer "F.Cu") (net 1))
 (segment (start 150.75 95.315) (end 150.75 93.8) (width 0.2) (layer "F.Cu") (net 1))
 (segment (start 150.25 94.3) (end 149.5 93.55) (width 0.2) (layer "F.Cu") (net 1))
 (segment (start 150.25 95.315) (end 150.25 94.3) (width 0.2) (layer "F.Cu") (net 1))
 (segment (start 150.25 93.05) (end 150.5 93.05) (width 0.2) (layer "F.Cu") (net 1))
 (segment (start 149.75 93.55) (end 150.25 93.05) (width 0.2) (layer "F.Cu") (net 1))
 (via (at 150.25 93.05) (size 0.5) (drill 0.2) (layers "F.Cu" "B.Cu") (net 1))
 (segment (start 150.65 100.45) (end 150.65 99.6) (width 0.5) (layer "B.Cu") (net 1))
 (segment (start 150.65 99.6) (end 150.65 100.3) (width 0.5) (layer "B.Cu") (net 1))
 (segment (start 158.6 98.5) (end 156.55 98.5) (width 0.5) (layer "B.Cu") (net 1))
 (segment (start 144.25 98.5) (end 142.4 98.5) (width 0.5) (layer "B.Cu") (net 1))
 (segment (start 146.223 100.473) (end 144.25 98.5) (width 0.5) (layer "B.Cu") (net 1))
 (segment (start 150.477 100.473) (end 146.223 100.473) (width 0.5) (layer "B.Cu") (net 1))
 (segment (start 156.55 98.5) (end 154.577 100.473) (width 0.5) (layer "B.Cu") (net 1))
 (segment (start 150.673 100.473) (end 150.65 100.45) (width 0.5) (layer "B.Cu") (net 1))
 (segment (start 154.577 100.473) (end 150.673 100.473) (width 0.5) (layer "B.Cu") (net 1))
 (segment (start 150.65 93.45) (end 150.25 93.05) (width 0.5) (layer "B.Cu") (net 1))
 (segment (start 150.65 99.6) (end 150.65 93.45) (width 0.5) (layer "B.Cu") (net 1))
 (segment (start 150.65 100.3) (end 150.477 100.473) (width 0.5) (layer "B.Cu") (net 1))
 (segment (start 151.638 95.703) (end 151.25 95.315) (width 0.2) (layer "F.Cu") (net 16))
 (segment (start 156.231224 97.096) (end 154.046 97.096) (width 0.2) (layer "F.Cu") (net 16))
 (segment (start 154.046 97.096) (end 152.8 95.85) (width 0.2) (layer "F.Cu") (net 16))
 (segment (start 151.944 95.85) (end 151.797 95.703) (width 0.2) (layer "F.Cu") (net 16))
 (segment (start 156.827224 96.5) (end 156.231224 97.096) (width 0.2) (layer "F.Cu") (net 16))
 (segment (start 151.797 95.703) (end 151.638 95.703) (width 0.2) (layer "F.Cu") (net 16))
 (segment (start 152.8 95.85) (end 151.944 95.85) (width 0.2) (layer "F.Cu") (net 16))
 (segment (start 158.65 96.5) (end 156.827224 96.5) (width 0.2) (layer "F.Cu") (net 16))
 (segment (start 153.873 97.423) (end 152.7 96.25) (width 0.2) (layer "F.Cu") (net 15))
 (segment (start 156.223 97.423) (end 153.873 97.423) (width 0.2) (layer "F.Cu") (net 15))
 (segment (start 158.65 98.5) (end 157.3 98.5) (width 0.2) (layer "F.Cu") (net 15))
 (segment (start 157.3 98.5) (end 156.223 97.423) (width 0.2) (layer "F.Cu") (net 15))
 (segment (start 152.7 96.25) (end 152.185 96.25) (width 0.2) (layer "F.Cu") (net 15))
 (segment (start 158.65 100.5) (end 157.75 100.5) (width 0.2) (layer "F.Cu") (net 12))
 (segment (start 156.673 98.335448) (end 156.087552 97.75) (width 0.2) (layer "F.Cu") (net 12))
 (segment (start 156.087552 97.75) (end 152.185 97.75) (width 0.2) (layer "F.Cu") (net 12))
 (segment (start 157.75 100.5) (end 156.673 99.423) (width 0.2) (layer "F.Cu") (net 12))
 (segment (start 156.673 99.423) (end 156.673 98.335448) (width 0.2) (layer "F.Cu") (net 12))
 (segment (start 154.6 98.15) (end 154.7 98.25) (width 0.2) (layer "F.Cu") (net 11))
 (segment (start 151.803 98.297) (end 151.95 98.15) (width 0.2) (layer "F.Cu") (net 11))
 (segment (start 151.25 98.685) (end 151.25 98.6) (width 0.2) (layer "F.Cu") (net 11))
 (segment (start 151.95 98.15) (end 154.6 98.15) (width 0.2) (layer "F.Cu") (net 11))
 (segment (start 151.553 98.297) (end 151.803 98.297) (width 0.2) (layer "F.Cu") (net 11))
 (segment (start 151.25 98.6) (end 151.553 98.297) (width 0.2) (layer "F.Cu") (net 11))
 (via (at 154.7 98.25) (size 0.5) (drill 0.2) (layers "F.Cu" "B.Cu") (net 11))
 (segment (start 155 97.95) (end 155 93.95) (width 0.2) (layer "B.Cu") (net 11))
 (segment (start 154.7 98.25) (end 155 97.95) (width 0.2) (layer "B.Cu") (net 11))
 (segment (start 156.45 92.5) (end 158.6 92.5) (width 0.2) (layer "B.Cu") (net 11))
 (segment (start 155 93.95) (end 156.45 92.5) (width 0.2) (layer "B.Cu") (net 11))
 (segment (start 142.35 100.5) (end 143.45 100.5) (width 0.2) (layer "F.Cu") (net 6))
 (segment (start 145.4 95.2) (end 149.635 95.2) (width 0.2) (layer "F.Cu") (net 6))
 (segment (start 143.45 100.5) (end 144.8 99.15) (width 0.2) (layer "F.Cu") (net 6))
 (segment (start 149.635 95.2) (end 149.75 95.315) (width 0.2) (layer "F.Cu") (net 6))
 (segment (start 145.386937 98.563063) (end 145.386937 97.286937) (width 0.2) (layer "F.Cu") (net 6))
 (segment (start 144.8 99.15) (end 145.386937 98.563063) (width 0.2) (layer "F.Cu") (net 6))
 (via (at 145.4 95.2) (size 0.5) (drill 0.2) (layers "F.Cu" "B.Cu") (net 6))
 (via (at 145.386937 97.286937) (size 0.5) (drill 0.2) (layers "F.Cu" "B.Cu") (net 6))
 (segment (start 145.4 97.273874) (end 145.4 95.2) (width 0.2) (layer "B.Cu") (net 6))
 (segment (start 145.386937 97.286937) (end 145.4 97.273874) (width 0.2) (layer "B.Cu") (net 6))
 (segment (start 145.15 101.1) (end 144.55 100.5) (width 0.5) (layer "B.Cu") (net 10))
 (segment (start 155.6 101.1) (end 145.15 101.1) (width 0.5) (layer "B.Cu") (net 10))
 (segment (start 156.2 100.5) (end 155.6 101.1) (width 0.5) (layer "B.Cu") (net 10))
 (segment (start 144.55 100.5) (end 142.3 100.5) (width 0.5) (layer "B.Cu") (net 10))
 (segment (start 158.5 100.5) (end 156.2 100.5) (width 0.5) (layer "B.Cu") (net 10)))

